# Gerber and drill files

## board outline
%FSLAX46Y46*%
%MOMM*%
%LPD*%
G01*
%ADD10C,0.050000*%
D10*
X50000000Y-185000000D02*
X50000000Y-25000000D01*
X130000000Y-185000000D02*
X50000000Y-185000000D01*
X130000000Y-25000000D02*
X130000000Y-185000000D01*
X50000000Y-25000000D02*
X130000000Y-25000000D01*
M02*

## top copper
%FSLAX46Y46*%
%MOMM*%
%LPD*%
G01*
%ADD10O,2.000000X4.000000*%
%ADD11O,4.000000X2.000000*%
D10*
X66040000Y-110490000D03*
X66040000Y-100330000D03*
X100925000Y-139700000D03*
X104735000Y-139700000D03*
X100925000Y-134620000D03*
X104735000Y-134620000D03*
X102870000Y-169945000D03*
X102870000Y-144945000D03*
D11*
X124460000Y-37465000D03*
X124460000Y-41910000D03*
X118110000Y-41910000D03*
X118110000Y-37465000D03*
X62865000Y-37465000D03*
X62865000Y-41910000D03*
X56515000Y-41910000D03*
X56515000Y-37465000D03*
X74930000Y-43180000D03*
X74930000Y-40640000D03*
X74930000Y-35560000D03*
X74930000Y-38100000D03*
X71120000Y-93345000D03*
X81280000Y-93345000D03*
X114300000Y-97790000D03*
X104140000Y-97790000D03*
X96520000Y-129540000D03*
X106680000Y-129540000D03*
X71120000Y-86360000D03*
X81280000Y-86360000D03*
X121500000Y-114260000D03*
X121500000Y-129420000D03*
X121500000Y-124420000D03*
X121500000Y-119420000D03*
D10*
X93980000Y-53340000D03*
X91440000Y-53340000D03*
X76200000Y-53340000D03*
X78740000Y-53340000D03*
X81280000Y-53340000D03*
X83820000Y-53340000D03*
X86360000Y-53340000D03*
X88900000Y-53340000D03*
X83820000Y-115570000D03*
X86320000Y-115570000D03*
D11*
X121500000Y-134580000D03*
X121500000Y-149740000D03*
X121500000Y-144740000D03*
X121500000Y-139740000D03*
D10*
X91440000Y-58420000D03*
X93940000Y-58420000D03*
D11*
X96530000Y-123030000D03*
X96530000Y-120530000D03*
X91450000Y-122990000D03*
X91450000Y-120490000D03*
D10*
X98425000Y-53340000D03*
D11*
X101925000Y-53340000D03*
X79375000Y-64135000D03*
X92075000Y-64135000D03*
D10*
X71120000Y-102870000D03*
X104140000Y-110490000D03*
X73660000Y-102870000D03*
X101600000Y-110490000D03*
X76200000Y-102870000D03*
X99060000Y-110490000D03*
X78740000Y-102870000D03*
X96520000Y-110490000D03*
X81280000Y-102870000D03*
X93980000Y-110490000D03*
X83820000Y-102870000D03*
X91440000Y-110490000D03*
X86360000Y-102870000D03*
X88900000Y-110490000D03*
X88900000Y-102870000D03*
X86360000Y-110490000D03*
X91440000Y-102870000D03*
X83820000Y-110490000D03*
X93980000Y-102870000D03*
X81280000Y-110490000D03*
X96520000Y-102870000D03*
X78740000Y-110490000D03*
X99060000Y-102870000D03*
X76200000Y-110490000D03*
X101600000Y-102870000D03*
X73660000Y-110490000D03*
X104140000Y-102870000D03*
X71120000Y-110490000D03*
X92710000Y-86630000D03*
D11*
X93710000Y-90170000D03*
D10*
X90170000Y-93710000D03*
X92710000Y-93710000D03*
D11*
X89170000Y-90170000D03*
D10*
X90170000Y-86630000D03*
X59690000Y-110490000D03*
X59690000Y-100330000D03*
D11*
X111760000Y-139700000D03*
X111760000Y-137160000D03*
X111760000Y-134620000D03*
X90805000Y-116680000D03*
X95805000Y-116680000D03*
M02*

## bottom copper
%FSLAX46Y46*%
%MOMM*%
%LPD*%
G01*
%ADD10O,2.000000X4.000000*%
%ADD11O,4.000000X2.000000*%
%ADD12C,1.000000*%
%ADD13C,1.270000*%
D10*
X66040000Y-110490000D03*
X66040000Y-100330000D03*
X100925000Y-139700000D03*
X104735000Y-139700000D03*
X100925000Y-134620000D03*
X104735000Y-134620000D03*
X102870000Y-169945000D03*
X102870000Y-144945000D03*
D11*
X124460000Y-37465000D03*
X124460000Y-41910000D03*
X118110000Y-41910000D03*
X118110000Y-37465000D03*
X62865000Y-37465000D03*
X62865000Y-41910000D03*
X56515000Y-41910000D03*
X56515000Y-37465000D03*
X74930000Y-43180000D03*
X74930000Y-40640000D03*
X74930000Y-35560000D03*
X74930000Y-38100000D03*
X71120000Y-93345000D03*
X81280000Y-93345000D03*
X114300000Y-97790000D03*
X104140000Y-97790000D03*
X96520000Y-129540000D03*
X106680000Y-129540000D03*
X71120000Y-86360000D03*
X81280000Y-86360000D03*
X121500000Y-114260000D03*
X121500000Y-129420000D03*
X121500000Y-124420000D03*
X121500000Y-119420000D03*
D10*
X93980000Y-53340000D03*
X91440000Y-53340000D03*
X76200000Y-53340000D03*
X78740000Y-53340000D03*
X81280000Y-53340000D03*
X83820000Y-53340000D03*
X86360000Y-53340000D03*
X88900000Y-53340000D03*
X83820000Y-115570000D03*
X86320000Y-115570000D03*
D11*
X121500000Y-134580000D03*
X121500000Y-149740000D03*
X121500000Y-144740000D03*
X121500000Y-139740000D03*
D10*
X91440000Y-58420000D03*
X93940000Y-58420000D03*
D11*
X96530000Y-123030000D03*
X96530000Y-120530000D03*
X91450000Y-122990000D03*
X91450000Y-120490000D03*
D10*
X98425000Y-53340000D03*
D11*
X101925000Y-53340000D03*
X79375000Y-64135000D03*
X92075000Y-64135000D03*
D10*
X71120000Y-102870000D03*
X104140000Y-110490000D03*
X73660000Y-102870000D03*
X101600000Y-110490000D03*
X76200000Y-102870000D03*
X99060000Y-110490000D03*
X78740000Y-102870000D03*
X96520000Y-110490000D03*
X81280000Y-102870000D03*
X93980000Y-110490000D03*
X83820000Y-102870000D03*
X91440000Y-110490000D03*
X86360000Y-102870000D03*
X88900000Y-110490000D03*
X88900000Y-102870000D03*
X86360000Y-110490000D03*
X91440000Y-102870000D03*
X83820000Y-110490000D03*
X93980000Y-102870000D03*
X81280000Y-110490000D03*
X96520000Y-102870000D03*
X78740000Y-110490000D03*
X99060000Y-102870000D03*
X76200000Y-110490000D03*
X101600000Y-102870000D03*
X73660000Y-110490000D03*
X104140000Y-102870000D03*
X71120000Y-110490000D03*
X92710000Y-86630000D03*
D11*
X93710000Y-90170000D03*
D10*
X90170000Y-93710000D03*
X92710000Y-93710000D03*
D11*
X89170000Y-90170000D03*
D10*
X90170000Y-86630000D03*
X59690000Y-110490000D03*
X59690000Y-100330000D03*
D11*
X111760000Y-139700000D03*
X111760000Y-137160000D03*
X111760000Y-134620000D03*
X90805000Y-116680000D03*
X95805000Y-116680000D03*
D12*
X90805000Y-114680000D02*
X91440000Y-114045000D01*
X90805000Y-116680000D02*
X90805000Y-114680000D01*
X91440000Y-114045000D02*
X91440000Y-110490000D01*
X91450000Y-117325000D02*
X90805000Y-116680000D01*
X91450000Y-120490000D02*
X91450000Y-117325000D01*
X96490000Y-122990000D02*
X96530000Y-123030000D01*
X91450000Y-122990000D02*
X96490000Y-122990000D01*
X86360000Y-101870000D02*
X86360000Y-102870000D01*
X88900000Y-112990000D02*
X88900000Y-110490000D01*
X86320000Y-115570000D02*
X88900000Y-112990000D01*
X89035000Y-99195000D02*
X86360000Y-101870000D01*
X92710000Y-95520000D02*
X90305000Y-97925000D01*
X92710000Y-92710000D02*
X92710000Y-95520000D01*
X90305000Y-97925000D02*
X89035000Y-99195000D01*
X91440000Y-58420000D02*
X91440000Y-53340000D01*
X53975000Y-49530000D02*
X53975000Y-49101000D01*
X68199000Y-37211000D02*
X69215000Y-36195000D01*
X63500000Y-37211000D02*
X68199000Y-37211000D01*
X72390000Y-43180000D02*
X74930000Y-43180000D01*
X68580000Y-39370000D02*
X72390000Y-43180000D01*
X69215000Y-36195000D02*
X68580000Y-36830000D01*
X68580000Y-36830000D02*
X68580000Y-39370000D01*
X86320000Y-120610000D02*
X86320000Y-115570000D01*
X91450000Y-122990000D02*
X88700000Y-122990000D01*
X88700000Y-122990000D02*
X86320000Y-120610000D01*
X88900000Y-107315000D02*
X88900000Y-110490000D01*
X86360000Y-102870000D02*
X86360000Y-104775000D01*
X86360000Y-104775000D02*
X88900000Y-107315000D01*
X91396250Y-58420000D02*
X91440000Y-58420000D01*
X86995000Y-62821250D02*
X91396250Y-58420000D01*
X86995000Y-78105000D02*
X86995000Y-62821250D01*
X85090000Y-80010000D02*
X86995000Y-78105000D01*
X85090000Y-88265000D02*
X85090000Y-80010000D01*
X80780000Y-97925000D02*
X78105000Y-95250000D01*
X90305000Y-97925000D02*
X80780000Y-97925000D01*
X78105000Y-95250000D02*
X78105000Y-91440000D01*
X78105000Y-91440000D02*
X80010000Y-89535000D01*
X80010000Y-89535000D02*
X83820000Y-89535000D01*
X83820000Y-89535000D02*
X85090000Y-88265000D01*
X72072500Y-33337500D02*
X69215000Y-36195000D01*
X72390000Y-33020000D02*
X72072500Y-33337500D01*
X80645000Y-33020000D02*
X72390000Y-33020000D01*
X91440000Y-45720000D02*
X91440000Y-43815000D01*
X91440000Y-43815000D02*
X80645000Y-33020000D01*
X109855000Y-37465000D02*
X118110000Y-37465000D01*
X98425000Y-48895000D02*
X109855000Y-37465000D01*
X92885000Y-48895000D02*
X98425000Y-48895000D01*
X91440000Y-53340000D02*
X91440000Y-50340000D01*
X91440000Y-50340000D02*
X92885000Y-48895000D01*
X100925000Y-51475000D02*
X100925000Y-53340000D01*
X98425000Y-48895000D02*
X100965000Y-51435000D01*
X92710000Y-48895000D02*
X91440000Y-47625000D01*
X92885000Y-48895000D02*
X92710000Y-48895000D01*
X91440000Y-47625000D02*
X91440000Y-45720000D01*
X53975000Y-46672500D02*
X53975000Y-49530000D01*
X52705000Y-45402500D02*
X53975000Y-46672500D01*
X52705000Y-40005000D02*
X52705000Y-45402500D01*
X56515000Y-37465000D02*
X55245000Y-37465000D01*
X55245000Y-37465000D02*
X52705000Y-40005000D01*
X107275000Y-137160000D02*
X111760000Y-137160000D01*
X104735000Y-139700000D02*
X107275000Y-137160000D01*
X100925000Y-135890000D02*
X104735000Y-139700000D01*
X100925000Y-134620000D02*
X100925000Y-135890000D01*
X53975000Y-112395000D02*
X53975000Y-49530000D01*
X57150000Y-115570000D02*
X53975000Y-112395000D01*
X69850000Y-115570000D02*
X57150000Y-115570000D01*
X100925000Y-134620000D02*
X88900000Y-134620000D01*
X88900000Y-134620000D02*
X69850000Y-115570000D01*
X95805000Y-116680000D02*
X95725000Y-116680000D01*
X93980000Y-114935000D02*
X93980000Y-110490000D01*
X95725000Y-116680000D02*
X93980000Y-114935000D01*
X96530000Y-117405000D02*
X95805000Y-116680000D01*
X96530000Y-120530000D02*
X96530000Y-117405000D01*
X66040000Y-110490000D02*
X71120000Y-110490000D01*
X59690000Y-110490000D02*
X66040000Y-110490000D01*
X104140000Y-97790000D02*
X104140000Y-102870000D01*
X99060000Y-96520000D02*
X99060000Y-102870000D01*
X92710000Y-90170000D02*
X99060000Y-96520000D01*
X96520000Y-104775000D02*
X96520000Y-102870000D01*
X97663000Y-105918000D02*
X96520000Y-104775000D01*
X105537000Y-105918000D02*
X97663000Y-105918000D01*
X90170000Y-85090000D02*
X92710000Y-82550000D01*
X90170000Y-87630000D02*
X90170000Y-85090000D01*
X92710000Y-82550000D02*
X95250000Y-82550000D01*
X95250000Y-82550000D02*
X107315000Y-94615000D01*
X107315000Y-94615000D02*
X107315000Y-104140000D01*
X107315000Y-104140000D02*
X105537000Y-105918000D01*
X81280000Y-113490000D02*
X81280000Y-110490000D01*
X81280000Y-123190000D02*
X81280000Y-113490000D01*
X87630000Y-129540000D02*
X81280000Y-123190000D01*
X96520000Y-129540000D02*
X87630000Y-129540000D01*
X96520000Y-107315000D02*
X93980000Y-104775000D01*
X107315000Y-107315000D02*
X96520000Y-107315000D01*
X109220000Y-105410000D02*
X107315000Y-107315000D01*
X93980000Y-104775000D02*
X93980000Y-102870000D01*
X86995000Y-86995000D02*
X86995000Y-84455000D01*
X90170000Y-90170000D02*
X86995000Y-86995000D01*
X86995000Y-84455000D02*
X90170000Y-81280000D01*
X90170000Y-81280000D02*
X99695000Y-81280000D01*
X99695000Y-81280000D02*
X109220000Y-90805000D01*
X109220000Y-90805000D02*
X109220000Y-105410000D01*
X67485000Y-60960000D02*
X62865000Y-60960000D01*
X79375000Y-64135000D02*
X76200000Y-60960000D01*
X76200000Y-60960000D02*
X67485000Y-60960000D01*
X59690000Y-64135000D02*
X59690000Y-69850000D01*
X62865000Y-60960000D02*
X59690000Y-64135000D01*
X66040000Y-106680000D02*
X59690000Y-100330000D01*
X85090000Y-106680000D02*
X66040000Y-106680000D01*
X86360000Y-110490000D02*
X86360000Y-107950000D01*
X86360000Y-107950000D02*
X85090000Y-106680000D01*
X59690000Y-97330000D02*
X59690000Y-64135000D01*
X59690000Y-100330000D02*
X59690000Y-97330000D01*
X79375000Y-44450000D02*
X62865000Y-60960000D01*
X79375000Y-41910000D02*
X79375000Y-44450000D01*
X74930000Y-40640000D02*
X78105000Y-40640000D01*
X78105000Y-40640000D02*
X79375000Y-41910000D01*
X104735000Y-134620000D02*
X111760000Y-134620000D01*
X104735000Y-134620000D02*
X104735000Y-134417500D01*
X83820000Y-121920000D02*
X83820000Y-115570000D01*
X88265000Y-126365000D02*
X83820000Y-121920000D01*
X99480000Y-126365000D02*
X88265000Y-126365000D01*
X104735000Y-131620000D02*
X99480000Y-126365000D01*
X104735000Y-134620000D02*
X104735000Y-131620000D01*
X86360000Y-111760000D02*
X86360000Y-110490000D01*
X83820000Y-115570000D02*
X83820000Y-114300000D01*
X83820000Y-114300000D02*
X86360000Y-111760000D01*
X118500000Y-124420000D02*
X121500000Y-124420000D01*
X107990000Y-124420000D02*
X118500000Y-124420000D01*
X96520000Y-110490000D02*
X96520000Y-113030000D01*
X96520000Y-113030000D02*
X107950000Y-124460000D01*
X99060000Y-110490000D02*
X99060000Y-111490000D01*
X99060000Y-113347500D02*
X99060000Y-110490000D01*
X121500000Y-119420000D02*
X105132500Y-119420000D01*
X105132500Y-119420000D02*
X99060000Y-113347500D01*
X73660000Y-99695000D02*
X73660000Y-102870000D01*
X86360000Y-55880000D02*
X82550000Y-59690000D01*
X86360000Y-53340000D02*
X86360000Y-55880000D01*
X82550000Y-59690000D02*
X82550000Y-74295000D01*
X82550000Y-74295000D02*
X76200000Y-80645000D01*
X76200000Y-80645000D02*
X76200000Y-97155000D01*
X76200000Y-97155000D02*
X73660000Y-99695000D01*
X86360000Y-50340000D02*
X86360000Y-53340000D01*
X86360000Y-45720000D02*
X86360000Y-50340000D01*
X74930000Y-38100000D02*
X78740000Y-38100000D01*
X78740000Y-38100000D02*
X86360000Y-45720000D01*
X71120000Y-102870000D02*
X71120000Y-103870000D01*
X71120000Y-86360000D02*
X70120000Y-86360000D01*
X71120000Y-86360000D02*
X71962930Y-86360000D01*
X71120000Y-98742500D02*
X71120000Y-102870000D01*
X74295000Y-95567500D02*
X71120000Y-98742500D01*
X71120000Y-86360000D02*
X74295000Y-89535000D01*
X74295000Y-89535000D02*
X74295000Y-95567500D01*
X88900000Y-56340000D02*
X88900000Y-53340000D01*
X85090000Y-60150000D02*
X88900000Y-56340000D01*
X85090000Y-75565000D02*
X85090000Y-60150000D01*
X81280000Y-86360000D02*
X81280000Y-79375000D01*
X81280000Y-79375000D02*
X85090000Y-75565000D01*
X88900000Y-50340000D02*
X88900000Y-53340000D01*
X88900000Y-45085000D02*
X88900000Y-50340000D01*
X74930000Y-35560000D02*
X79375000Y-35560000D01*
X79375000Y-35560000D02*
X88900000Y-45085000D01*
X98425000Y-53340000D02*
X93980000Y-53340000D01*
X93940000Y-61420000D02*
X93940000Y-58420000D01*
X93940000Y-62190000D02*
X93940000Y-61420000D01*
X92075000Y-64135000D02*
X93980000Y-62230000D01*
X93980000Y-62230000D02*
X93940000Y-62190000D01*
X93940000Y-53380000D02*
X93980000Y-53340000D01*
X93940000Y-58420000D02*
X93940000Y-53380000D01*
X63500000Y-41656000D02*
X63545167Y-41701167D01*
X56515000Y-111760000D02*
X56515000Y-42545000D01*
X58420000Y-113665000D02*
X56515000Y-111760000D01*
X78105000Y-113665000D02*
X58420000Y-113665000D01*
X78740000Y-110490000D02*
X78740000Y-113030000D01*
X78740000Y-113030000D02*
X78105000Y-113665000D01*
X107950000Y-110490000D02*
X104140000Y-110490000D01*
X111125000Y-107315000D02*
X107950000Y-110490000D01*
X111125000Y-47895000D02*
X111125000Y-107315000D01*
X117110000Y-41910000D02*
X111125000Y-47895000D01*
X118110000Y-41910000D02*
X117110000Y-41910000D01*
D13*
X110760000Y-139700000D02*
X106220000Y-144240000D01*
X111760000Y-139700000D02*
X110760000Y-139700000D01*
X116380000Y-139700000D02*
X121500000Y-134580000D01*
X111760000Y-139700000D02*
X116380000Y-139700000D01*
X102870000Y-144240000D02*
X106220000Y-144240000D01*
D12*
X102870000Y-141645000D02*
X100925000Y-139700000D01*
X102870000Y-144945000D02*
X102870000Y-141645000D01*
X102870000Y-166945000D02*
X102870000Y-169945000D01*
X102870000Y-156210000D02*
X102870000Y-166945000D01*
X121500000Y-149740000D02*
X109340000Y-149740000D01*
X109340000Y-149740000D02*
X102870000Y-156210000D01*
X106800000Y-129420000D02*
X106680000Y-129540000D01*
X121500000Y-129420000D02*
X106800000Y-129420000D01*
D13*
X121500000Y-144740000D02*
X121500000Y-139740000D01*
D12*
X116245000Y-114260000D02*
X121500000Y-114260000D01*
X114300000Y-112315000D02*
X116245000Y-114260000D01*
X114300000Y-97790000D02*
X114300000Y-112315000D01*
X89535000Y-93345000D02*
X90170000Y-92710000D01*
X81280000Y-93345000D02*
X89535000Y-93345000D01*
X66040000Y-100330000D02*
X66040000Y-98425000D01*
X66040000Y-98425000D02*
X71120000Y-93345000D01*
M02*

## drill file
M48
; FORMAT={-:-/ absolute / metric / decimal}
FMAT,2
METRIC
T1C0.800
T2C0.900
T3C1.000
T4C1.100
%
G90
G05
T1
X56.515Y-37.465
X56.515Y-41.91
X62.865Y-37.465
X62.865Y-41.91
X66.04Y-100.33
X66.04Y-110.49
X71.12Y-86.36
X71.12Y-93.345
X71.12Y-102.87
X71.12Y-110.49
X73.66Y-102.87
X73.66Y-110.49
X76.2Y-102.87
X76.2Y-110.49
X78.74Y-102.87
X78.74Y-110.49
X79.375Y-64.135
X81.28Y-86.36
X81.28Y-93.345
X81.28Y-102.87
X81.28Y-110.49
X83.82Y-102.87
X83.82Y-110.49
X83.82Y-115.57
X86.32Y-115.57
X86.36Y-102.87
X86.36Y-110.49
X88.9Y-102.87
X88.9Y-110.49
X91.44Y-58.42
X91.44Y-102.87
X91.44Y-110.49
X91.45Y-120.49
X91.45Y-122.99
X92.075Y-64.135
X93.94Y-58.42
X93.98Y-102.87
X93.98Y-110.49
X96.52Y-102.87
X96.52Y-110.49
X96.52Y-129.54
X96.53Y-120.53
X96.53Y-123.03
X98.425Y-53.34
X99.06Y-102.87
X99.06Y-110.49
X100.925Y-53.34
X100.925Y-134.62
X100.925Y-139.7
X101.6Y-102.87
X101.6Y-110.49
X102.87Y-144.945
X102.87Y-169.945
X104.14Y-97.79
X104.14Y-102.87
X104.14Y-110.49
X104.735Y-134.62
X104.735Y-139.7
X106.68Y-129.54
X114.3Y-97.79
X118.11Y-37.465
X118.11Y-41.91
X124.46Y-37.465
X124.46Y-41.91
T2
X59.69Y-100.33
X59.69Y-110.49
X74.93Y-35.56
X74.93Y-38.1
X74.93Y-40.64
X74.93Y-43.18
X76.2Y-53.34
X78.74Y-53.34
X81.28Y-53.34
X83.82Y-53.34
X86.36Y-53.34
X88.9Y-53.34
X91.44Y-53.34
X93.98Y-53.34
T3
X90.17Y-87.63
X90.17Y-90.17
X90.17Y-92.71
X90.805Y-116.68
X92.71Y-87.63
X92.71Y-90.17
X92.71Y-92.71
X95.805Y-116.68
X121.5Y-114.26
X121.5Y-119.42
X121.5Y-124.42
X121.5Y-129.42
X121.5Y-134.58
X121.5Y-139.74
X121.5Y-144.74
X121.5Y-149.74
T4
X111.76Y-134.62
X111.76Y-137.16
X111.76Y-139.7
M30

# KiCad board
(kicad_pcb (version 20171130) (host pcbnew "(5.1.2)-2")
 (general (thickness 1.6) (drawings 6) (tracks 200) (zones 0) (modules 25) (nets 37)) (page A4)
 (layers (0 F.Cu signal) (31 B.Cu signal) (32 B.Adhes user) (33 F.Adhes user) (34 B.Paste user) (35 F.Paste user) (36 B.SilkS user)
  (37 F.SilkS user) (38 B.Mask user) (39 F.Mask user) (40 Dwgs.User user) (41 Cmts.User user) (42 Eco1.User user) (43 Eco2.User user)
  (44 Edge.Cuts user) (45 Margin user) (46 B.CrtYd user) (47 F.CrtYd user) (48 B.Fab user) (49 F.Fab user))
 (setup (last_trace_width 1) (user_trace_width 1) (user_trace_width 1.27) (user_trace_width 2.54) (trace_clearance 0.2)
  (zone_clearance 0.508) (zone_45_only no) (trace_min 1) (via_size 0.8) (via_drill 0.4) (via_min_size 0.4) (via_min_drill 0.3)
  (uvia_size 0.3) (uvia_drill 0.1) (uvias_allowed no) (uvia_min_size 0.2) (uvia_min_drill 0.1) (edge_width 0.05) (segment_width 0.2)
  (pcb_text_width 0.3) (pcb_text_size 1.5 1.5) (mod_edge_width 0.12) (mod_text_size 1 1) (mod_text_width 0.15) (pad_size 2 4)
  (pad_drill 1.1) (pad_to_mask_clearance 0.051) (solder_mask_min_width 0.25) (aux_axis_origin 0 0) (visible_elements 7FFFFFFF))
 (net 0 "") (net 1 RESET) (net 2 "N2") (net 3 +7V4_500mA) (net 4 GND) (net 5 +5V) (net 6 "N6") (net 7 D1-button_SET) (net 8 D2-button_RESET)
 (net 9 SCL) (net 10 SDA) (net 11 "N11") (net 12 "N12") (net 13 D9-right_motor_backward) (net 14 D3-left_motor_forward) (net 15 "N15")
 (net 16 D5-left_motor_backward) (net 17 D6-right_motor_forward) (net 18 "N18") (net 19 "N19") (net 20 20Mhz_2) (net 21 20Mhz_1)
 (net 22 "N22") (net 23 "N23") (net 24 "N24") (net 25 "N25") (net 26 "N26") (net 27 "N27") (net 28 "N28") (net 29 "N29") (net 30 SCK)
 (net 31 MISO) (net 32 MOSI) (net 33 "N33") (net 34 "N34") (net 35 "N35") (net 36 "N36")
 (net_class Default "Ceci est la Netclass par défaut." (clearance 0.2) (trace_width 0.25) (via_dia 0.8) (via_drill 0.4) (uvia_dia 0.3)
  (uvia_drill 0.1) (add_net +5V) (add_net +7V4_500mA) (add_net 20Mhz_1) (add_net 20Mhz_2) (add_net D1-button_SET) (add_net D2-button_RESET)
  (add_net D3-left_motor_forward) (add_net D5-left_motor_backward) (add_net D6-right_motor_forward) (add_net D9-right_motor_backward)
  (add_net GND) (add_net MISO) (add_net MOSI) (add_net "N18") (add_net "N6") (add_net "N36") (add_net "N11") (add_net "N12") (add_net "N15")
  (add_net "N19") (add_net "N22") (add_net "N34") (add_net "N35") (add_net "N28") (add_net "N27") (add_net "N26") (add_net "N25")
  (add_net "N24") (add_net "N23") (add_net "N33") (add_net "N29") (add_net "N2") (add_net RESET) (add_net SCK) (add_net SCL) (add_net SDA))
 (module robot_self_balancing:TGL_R (layer F.Cu) (at 66.04 100.33 270)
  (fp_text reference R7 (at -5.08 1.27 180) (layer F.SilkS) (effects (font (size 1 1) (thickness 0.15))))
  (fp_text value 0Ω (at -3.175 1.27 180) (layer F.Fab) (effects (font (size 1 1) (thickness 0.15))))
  (pad 2 thru_hole oval (at 10.16 0 270) (size 4 2) (drill 0.8) (layers *.Cu *.Mask) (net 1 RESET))
  (pad 1 thru_hole oval (at 0 0 270) (size 4 2) (drill 0.8) (layers *.Cu *.Mask) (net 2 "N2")))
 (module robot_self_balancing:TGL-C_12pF (layer F.Cu) (at 104.1 139.7 180)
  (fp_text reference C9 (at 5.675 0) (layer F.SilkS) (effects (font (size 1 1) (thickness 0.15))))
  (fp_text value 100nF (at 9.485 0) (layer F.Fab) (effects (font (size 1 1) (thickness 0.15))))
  (pad 2 thru_hole oval (at 3.175 0 180) (size 2 4) (drill 0.8) (layers *.Cu *.Mask) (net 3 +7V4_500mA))
  (pad 1 thru_hole oval (at -0.635 0 180) (size 2 4) (drill 0.8) (layers *.Cu *.Mask) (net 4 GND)))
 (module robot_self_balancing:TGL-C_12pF (layer F.Cu) (at 104.1 134.62 180)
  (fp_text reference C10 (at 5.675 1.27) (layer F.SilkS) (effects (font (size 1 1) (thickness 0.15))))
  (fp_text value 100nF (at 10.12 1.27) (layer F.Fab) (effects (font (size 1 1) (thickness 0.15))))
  (pad 2 thru_hole oval (at 3.175 0 180) (size 2 4) (drill 0.8) (layers *.Cu *.Mask) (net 4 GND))
  (pad 1 thru_hole oval (at -0.635 0 180) (size 2 4) (drill 0.8) (layers *.Cu *.Mask) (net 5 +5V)))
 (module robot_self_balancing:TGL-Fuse (layer F.Cu) (at 111.76 156.845 270)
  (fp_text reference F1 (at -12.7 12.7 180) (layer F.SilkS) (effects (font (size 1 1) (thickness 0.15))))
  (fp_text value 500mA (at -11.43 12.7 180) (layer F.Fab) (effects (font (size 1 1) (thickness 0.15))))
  (pad 2 thru_hole oval (at 13.1 8.89 270) (size 4 2) (drill 0.8) (layers *.Cu *.Mask) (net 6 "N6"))
  (pad 1 thru_hole oval (at -11.9 8.89 270) (size 4 2) (drill 0.8) (layers *.Cu *.Mask) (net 3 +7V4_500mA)))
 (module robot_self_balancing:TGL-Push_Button (layer F.Cu) (at 121.285 34.925)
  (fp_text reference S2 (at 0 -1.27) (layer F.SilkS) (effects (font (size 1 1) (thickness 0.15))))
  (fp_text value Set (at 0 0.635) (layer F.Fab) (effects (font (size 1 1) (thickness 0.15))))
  (pad 1 thru_hole oval (at 3.175 2.54) (size 4 2) (drill 0.8) (layers *.Cu *.Mask) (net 4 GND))
  (pad 2 thru_hole oval (at 3.175 6.985) (size 4 2) (drill 0.8) (layers *.Cu *.Mask) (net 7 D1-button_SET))
  (pad 2 thru_hole oval (at -3.175 6.985) (size 4 2) (drill 0.8) (layers *.Cu *.Mask) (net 7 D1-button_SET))
  (pad 1 thru_hole oval (at -3.175 2.54) (size 4 2) (drill 0.8) (layers *.Cu *.Mask) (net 4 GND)))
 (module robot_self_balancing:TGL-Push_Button (layer F.Cu) (at 59.69 34.925)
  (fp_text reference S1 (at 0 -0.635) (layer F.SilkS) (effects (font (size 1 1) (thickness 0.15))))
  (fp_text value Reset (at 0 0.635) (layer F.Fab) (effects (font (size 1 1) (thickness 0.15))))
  (pad 1 thru_hole oval (at 3.175 2.54) (size 4 2) (drill 0.8) (layers *.Cu *.Mask) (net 4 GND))
  (pad 2 thru_hole oval (at 3.175 6.985) (size 4 2) (drill 0.8) (layers *.Cu *.Mask) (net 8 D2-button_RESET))
  (pad 2 thru_hole oval (at -3.175 6.985) (size 4 2) (drill 0.8) (layers *.Cu *.Mask) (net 8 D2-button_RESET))
  (pad 1 thru_hole oval (at -3.175 2.54) (size 4 2) (drill 0.8) (layers *.Cu *.Mask) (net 4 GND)))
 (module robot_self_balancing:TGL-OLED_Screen (layer F.Cu) (at 71.12 39.37 90)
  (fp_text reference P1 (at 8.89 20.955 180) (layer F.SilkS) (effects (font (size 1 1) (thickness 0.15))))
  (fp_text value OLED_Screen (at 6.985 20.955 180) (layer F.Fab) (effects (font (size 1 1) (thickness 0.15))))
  (pad 1 thru_hole oval (at -3.81 3.81 90) (size 2 4) (drill 0.9) (layers *.Cu *.Mask) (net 4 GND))
  (pad 2 thru_hole oval (at -1.27 3.81 90) (size 2 4) (drill 0.9) (layers *.Cu *.Mask) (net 5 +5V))
  (pad 4 thru_hole oval (at 3.81 3.81 90) (size 2 4) (drill 0.9) (layers *.Cu *.Mask) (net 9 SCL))
  (pad 3 thru_hole oval (at 1.27 3.81 90) (size 2 4) (drill 0.9) (layers *.Cu *.Mask) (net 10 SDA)))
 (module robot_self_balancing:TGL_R (layer F.Cu) (at 81.28 93.345 180)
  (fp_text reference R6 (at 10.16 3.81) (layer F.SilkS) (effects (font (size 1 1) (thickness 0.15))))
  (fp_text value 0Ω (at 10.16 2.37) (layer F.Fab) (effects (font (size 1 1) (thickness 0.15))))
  (pad 2 thru_hole oval (at 10.16 0 180) (size 4 2) (drill 0.8) (layers *.Cu *.Mask) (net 2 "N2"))
  (pad 1 thru_hole oval (at 0 0 180) (size 4 2) (drill 0.8) (layers *.Cu *.Mask) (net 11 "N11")))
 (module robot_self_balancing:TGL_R (layer F.Cu) (at 104.14 97.79)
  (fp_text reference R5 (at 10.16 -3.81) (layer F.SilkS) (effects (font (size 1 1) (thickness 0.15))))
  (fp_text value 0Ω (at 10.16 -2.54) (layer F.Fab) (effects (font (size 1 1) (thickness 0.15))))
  (pad 2 thru_hole oval (at 10.16 0) (size 4 2) (drill 0.8) (layers *.Cu *.Mask) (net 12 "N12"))
  (pad 1 thru_hole oval (at 0 0) (size 4 2) (drill 0.8) (layers *.Cu *.Mask) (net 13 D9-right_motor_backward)))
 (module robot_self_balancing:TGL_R (layer F.Cu) (at 106.68 129.54 180)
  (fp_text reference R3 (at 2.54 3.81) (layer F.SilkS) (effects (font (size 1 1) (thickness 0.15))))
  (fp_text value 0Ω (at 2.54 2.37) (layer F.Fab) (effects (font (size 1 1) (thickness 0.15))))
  (pad 2 thru_hole oval (at 10.16 0 180) (size 4 2) (drill 0.8) (layers *.Cu *.Mask) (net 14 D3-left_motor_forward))
  (pad 1 thru_hole oval (at 0 0 180) (size 4 2) (drill 0.8) (layers *.Cu *.Mask) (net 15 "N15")))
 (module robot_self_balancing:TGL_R (layer F.Cu) (at 81.28 86.36 180)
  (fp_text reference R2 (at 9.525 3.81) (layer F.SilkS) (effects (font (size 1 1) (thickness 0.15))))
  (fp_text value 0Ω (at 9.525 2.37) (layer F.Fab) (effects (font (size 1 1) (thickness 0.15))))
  (pad 2 thru_hole oval (at 10.16 0 180) (size 4 2) (drill 0.8) (layers *.Cu *.Mask) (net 9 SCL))
  (pad 1 thru_hole oval (at 0 0 180) (size 4 2) (drill 0.8) (layers *.Cu *.Mask) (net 9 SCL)))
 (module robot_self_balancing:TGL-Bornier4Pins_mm (layer F.Cu) (at 127 121.92 270)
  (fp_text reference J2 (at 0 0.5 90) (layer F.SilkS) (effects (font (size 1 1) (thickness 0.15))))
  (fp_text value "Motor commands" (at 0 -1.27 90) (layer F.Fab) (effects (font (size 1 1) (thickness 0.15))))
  (pad 5 thru_hole oval (at -7.66 5.5 270) (size 2 4) (drill 1) (layers *.Cu *.Mask) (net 12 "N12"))
  (pad 8 thru_hole oval (at 7.5 5.5 90) (size 2 4) (drill 1) (layers *.Cu *.Mask) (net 15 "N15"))
  (pad 7 thru_hole oval (at 2.5 5.5 270) (size 2 4) (drill 1) (layers *.Cu *.Mask) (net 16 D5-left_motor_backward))
  (pad 6 thru_hole oval (at -2.5 5.5 270) (size 2 4) (drill 1) (layers *.Cu *.Mask) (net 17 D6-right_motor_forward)))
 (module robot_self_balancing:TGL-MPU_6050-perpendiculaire (layer F.Cu) (at 85.09 57.15 180)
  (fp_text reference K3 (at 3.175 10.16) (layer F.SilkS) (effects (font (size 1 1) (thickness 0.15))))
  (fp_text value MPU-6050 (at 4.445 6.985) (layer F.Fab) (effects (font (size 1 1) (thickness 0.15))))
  (pad 13 thru_hole oval (at -8.89 3.81 180) (size 2 4) (drill 0.9) (layers *.Cu *.Mask) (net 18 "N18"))
  (pad 18 thru_hole oval (at -6.35 3.81 180) (size 2 4) (drill 0.9) (layers *.Cu *.Mask) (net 4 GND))
  (pad "" thru_hole oval (at 8.89 3.81 180) (size 2 4) (drill 0.9) (layers *.Cu *.Mask))
  (pad "" thru_hole oval (at 6.35 3.81 180) (size 2 4) (drill 0.9) (layers *.Cu *.Mask))
  (pad "" thru_hole oval (at 3.81 3.81 180) (size 2 4) (drill 0.9) (layers *.Cu *.Mask))
  (pad "" thru_hole oval (at 1.27 3.81 180) (size 2 4) (drill 0.9) (layers *.Cu *.Mask))
  (pad 24 thru_hole oval (at -1.27 3.81 180) (size 2 4) (drill 0.9) (layers *.Cu *.Mask) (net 10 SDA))
  (pad 23 thru_hole oval (at -3.81 3.81 180) (size 2 4) (drill 0.9) (layers *.Cu *.Mask) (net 9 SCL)))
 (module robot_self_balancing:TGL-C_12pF (layer F.Cu) (at 86.32 115.57 180)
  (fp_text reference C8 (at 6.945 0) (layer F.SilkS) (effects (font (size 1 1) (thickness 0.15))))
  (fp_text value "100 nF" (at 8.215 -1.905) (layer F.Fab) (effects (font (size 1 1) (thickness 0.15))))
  (pad 2 thru_hole oval (at 2.5 0 180) (size 2 4) (drill 0.8) (layers *.Cu *.Mask) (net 5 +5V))
  (pad 1 thru_hole oval (at 0 0 180) (size 2 4) (drill 0.8) (layers *.Cu *.Mask) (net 4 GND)))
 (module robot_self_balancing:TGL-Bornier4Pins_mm (layer F.Cu) (at 127 142.24 270)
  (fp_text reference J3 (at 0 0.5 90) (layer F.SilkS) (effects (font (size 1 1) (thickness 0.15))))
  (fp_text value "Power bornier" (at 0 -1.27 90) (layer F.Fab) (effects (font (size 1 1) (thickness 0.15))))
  (pad 8 thru_hole oval (at -7.66 5.5 270) (size 2 4) (drill 1) (layers *.Cu *.Mask) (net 3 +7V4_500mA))
  (pad 5 thru_hole oval (at 7.5 5.5 90) (size 2 4) (drill 1) (layers *.Cu *.Mask) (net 6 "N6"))
  (pad 7 thru_hole oval (at 2.5 5.5 270) (size 2 4) (drill 1) (layers *.Cu *.Mask) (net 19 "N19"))
  (pad 6 thru_hole oval (at -2.5 5.5 270) (size 2 4) (drill 1) (layers *.Cu *.Mask) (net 19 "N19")))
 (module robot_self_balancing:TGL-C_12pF (layer F.Cu) (at 93.94 58.42 180)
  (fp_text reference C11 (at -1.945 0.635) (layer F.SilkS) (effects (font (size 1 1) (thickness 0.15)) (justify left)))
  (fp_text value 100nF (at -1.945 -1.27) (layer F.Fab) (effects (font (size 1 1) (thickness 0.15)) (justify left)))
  (pad 2 thru_hole oval (at 2.5 0 180) (size 2 4) (drill 0.8) (layers *.Cu *.Mask) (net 4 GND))
  (pad 1 thru_hole oval (at 0 0 180) (size 2 4) (drill 0.8) (layers *.Cu *.Mask) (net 18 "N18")))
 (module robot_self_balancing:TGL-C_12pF (layer F.Cu) (at 96.53 120.53 270)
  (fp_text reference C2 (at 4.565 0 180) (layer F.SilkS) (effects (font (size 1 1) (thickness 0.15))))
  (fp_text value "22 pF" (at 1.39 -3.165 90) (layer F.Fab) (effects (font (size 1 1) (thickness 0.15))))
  (pad 2 thru_hole oval (at 2.5 0 270) (size 2 4) (drill 0.8) (layers *.Cu *.Mask) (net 4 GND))
  (pad 1 thru_hole oval (at 0 0 270) (size 2 4) (drill 0.8) (layers *.Cu *.Mask) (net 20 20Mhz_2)))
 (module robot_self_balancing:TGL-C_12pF (layer F.Cu) (at 91.45 120.49 270)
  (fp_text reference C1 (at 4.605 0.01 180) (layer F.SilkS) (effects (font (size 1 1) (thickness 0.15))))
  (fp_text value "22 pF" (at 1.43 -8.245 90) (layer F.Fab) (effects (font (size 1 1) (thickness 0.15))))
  (pad 2 thru_hole oval (at 2.5 0 270) (size 2 4) (drill 0.8) (layers *.Cu *.Mask) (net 4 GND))
  (pad 1 thru_hole oval (at 0 0 270) (size 2 4) (drill 0.8) (layers *.Cu *.Mask) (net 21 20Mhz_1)))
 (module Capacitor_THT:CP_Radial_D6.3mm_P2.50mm (layer F.Cu) (at 98.425 53.34)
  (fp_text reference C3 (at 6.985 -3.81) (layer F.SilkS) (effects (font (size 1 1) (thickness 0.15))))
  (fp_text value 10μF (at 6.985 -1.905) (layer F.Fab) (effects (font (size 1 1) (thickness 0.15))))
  (pad 1 thru_hole oval (at 0 0) (size 2 4) (drill 0.8) (layers *.Cu *.Mask) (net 18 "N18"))
  (pad 2 thru_hole oval (at 2.5 0) (size 4 2) (drill 0.8 (offset 1 0)) (layers *.Cu *.Mask) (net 4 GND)))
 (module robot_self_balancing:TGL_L (layer F.Cu) (at 92.075 64.135 180)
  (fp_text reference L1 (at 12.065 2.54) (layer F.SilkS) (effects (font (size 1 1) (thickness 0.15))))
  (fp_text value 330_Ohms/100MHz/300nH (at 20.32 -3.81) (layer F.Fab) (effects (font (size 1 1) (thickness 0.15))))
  (pad 2 thru_hole oval (at 12.7 0 180) (size 4 2) (drill 0.8) (layers *.Cu *.Mask) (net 5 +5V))
  (pad 1 thru_hole oval (at 0 0 180) (size 4 2) (drill 0.8) (layers *.Cu *.Mask) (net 18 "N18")))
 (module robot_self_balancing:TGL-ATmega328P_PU (layer F.Cu) (at 71.12 110.49 90)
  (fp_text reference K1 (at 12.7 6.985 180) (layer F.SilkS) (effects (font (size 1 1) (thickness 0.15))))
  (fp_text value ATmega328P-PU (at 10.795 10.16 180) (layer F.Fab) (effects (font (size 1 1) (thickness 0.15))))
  (pad 28 thru_hole oval (at 7.62 0 90) (size 4 2) (drill 0.8) (layers *.Cu *.Mask) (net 9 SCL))
  (pad 14 thru_hole oval (at 0 33.02 90) (size 4 2) (drill 0.8) (layers *.Cu *.Mask) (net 7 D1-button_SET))
  (pad 27 thru_hole oval (at 7.62 2.54 90) (size 4 2) (drill 0.8) (layers *.Cu *.Mask) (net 10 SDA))
  (pad 13 thru_hole oval (at 0 30.48 90) (size 4 2) (drill 0.8) (layers *.Cu *.Mask) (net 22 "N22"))
  (pad 26 thru_hole oval (at 7.62 5.08 90) (size 4 2) (drill 0.8) (layers *.Cu *.Mask) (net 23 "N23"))
  (pad 12 thru_hole oval (at 0 27.94 90) (size 4 2) (drill 0.8) (layers *.Cu *.Mask) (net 17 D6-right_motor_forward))
  (pad 25 thru_hole oval (at 7.62 7.62 90) (size 4 2) (drill 0.8) (layers *.Cu *.Mask) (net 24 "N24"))
  (pad 11 thru_hole oval (at 0 25.4 90) (size 4 2) (drill 0.8) (layers *.Cu *.Mask) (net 16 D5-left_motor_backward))
  (pad 24 thru_hole oval (at 7.62 10.16 90) (size 4 2) (drill 0.8) (layers *.Cu *.Mask) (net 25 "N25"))
  (pad 10 thru_hole oval (at 0 22.86 90) (size 4 2) (drill 0.8) (layers *.Cu *.Mask) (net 20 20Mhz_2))
  (pad 23 thru_hole oval (at 7.62 12.7 90) (size 4 2) (drill 0.8) (layers *.Cu *.Mask) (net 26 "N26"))
  (pad 9 thru_hole oval (at 0 20.32 90) (size 4 2) (drill 0.8) (layers *.Cu *.Mask) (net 21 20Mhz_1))
  (pad 22 thru_hole oval (at 7.62 15.24 90) (size 4 2) (drill 0.8) (layers *.Cu *.Mask) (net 4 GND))
  (pad 8 thru_hole oval (at 0 17.78 90) (size 4 2) (drill 0.8) (layers *.Cu *.Mask) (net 4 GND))
  (pad 21 thru_hole oval (at 7.62 17.78 90) (size 4 2) (drill 0.8) (layers *.Cu *.Mask) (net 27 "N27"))
  (pad 7 thru_hole oval (at 0 15.24 90) (size 4 2) (drill 0.8) (layers *.Cu *.Mask) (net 5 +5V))
  (pad 20 thru_hole oval (at 7.62 20.32 90) (size 4 2) (drill 0.8) (layers *.Cu *.Mask) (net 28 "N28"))
  (pad 6 thru_hole oval (at 0 12.7 90) (size 4 2) (drill 0.8) (layers *.Cu *.Mask) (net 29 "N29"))
  (pad 19 thru_hole oval (at 7.62 22.86 90) (size 4 2) (drill 0.8) (layers *.Cu *.Mask) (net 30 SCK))
  (pad 5 thru_hole oval (at 0 10.16 90) (size 4 2) (drill 0.8) (layers *.Cu *.Mask) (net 14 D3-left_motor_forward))
  (pad 18 thru_hole oval (at 7.62 25.4 90) (size 4 2) (drill 0.8) (layers *.Cu *.Mask) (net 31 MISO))
  (pad 4 thru_hole oval (at 0 7.62 90) (size 4 2) (drill 0.8) (layers *.Cu *.Mask) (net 8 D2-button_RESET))
  (pad 17 thru_hole oval (at 7.62 27.94 90) (size 4 2) (drill 0.8) (layers *.Cu *.Mask) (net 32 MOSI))
  (pad 3 thru_hole oval (at 0 5.08 90) (size 4 2) (drill 0.8) (layers *.Cu *.Mask) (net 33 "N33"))
  (pad 16 thru_hole oval (at 7.62 30.48 90) (size 4 2) (drill 0.8) (layers *.Cu *.Mask) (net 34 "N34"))
  (pad 2 thru_hole oval (at 0 2.54 90) (size 4 2) (drill 0.8) (layers *.Cu *.Mask) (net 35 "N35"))
  (pad 15 thru_hole oval (at 7.62 33.02 90) (size 4 2) (drill 0.8) (layers *.Cu *.Mask) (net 13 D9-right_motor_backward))
  (pad 1 thru_hole oval (at 0 0 90) (size 4 2) (drill 0.8) (layers *.Cu *.Mask) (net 1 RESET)))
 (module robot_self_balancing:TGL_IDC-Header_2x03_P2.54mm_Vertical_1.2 (layer F.Cu) (at 90.17 87.63)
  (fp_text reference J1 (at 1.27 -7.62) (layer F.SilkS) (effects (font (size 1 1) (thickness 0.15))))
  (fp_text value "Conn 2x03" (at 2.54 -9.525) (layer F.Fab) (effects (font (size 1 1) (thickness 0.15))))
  (pad 2 thru_hole oval (at 2.54 0) (size 2 4) (drill 1 (offset 0 -1)) (layers *.Cu *.Mask) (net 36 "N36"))
  (pad 4 thru_hole oval (at 2.54 2.54) (size 4 2) (drill 1 (offset 1 0)) (layers *.Cu *.Mask) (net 32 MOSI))
  (pad 5 thru_hole oval (at 0 5.08) (size 2 4) (drill 1 (offset 0 1)) (layers *.Cu *.Mask) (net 11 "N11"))
  (pad 6 thru_hole oval (at 2.54 5.08) (size 2 4) (drill 1 (offset 0 1)) (layers *.Cu *.Mask) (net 4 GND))
  (pad 3 thru_hole oval (at 0 2.54) (size 4 2) (drill 1 (offset -1 0)) (layers *.Cu *.Mask) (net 30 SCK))
  (pad 1 thru_hole oval (at 0 0) (size 2 4) (drill 1 (offset 0 -1)) (layers *.Cu *.Mask) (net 31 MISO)))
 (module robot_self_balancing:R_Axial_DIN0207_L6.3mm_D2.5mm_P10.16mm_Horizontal (layer F.Cu) (at 59.69 100.33 270)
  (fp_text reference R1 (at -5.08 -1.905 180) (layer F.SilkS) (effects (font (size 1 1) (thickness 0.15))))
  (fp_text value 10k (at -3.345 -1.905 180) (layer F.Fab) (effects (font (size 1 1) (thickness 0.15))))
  (pad 2 thru_hole oval (at 10.16 0 270) (size 4 2) (drill 0.9) (layers *.Cu *.Mask) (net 1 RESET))
  (pad 1 thru_hole oval (at 0 0 270) (size 4 2) (drill 0.9) (layers *.Cu *.Mask) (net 5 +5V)))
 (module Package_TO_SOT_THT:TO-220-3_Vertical (layer F.Cu) (at 111.76 139.7 90)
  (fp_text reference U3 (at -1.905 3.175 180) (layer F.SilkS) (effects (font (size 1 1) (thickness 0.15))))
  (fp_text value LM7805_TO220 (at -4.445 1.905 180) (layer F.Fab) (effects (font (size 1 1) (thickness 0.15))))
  (pad 1 thru_hole oval (at 0 0 90) (size 2 4) (drill 1.1) (layers *.Cu *.Mask) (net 3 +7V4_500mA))
  (pad 2 thru_hole oval (at 2.54 0 90) (size 2 4) (drill 1.1) (layers *.Cu *.Mask) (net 4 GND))
  (pad 3 thru_hole oval (at 5.08 0 90) (size 2 4) (drill 1.1) (layers *.Cu *.Mask) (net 5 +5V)))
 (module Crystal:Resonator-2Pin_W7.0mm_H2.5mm (layer F.Cu) (at 90.805 116.68)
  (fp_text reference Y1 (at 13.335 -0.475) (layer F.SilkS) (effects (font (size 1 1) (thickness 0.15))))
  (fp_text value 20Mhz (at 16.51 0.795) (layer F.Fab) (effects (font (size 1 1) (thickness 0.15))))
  (pad 1 thru_hole oval (at 0 0) (size 4 2) (drill 1) (layers *.Cu *.Mask) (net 21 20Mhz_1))
  (pad 2 thru_hole oval (at 5 0) (size 4 2) (drill 1) (layers *.Cu *.Mask) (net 20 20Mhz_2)))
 (gr_line (start 50 185) (end 50 25) (layer Edge.Cuts) (width 0.05))
 (gr_line (start 130 185) (end 50 185) (layer Edge.Cuts) (width 0.05))
 (gr_line (start 130 25) (end 130 185) (layer Edge.Cuts) (width 0.05))
 (gr_line (start 50 25) (end 130 25) (layer Edge.Cuts) (width 0.05))
 (segment (start 90.805 114.68) (end 91.44 114.045) (width 1) (layer B.Cu) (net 21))
 (segment (start 90.805 116.68) (end 90.805 114.68) (width 1) (layer B.Cu) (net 21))
 (segment (start 91.44 114.045) (end 91.44 110.49) (width 1) (layer B.Cu) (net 21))
 (segment (start 91.45 117.325) (end 90.805 116.68) (width 1) (layer B.Cu) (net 21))
 (segment (start 91.45 120.49) (end 91.45 117.325) (width 1) (layer B.Cu) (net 21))
 (segment (start 96.49 122.99) (end 96.53 123.03) (width 1) (layer B.Cu) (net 4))
 (segment (start 91.45 122.99) (end 96.49 122.99) (width 1) (layer B.Cu) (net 4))
 (segment (start 86.36 101.87) (end 86.36 102.87) (width 1) (layer B.Cu) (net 4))
 (segment (start 88.9 112.99) (end 88.9 110.49) (width 1) (layer B.Cu) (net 4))
 (segment (start 86.32 115.57) (end 88.9 112.99) (width 1) (layer B.Cu) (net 4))
 (segment (start 89.035 99.195) (end 86.36 101.87) (width 1) (layer B.Cu) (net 4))
 (segment (start 92.71 95.52) (end 90.305 97.925) (width 1) (layer B.Cu) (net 4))
 (segment (start 92.71 92.71) (end 92.71 95.52) (width 1) (layer B.Cu) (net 4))
 (segment (start 90.305 97.925) (end 89.035 99.195) (width 1) (layer B.Cu) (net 4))
 (segment (start 91.44 58.42) (end 91.44 53.34) (width 1) (layer B.Cu) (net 4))
 (segment (start 53.975 49.53) (end 53.975 49.101) (width 1) (layer B.Cu) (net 4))
 (segment (start 68.199 37.211) (end 69.215 36.195) (width 1) (layer B.Cu) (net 4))
 (segment (start 63.5 37.211) (end 68.199 37.211) (width 1) (layer B.Cu) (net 4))
 (segment (start 72.39 43.18) (end 74.93 43.18) (width 1) (layer B.Cu) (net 4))
 (segment (start 68.58 39.37) (end 72.39 43.18) (width 1) (layer B.Cu) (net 4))
 (segment (start 69.215 36.195) (end 68.58 36.83) (width 1) (layer B.Cu) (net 4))
 (segment (start 68.58 36.83) (end 68.58 39.37) (width 1) (layer B.Cu) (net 4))
 (segment (start 86.32 120.61) (end 86.32 115.57) (width 1) (layer B.Cu) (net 4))
 (segment (start 91.45 122.99) (end 88.7 122.99) (width 1) (layer B.Cu) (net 4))
 (segment (start 88.7 122.99) (end 86.32 120.61) (width 1) (layer B.Cu) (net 4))
 (segment (start 88.9 107.315) (end 88.9 110.49) (width 1) (layer B.Cu) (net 4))
 (segment (start 86.36 102.87) (end 86.36 104.775) (width 1) (layer B.Cu) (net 4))
 (segment (start 86.36 104.775) (end 88.9 107.315) (width 1) (layer B.Cu) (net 4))
 (segment (start 91.39625 58.42) (end 91.44 58.42) (width 1) (layer B.Cu) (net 4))
 (segment (start 86.995 62.82125) (end 91.39625 58.42) (width 1) (layer B.Cu) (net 4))
 (segment (start 86.995 78.105) (end 86.995 62.82125) (width 1) (layer B.Cu) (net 4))
 (segment (start 85.09 80.01) (end 86.995 78.105) (width 1) (layer B.Cu) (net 4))
 (segment (start 85.09 88.265) (end 85.09 80.01) (width 1) (layer B.Cu) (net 4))
 (segment (start 80.78 97.925) (end 78.105 95.25) (width 1) (layer B.Cu) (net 4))
 (segment (start 90.305 97.925) (end 80.78 97.925) (width 1) (layer B.Cu) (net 4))
 (segment (start 78.105 95.25) (end 78.105 91.44) (width 1) (layer B.Cu) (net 4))
 (segment (start 78.105 91.44) (end 80.01 89.535) (width 1) (layer B.Cu) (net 4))
 (segment (start 80.01 89.535) (end 83.82 89.535) (width 1) (layer B.Cu) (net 4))
 (segment (start 83.82 89.535) (end 85.09 88.265) (width 1) (layer B.Cu) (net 4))
 (segment (start 72.0725 33.3375) (end 69.215 36.195) (width 1) (layer B.Cu) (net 4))
 (segment (start 72.39 33.02) (end 72.0725 33.3375) (width 1) (layer B.Cu) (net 4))
 (segment (start 80.645 33.02) (end 72.39 33.02) (width 1) (layer B.Cu) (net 4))
 (segment (start 91.44 45.72) (end 91.44 43.815) (width 1) (layer B.Cu) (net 4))
 (segment (start 91.44 43.815) (end 80.645 33.02) (width 1) (layer B.Cu) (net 4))
 (segment (start 109.855 37.465) (end 118.11 37.465) (width 1) (layer B.Cu) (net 4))
 (segment (start 98.425 48.895) (end 109.855 37.465) (width 1) (layer B.Cu) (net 4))
 (segment (start 92.885 48.895) (end 98.425 48.895) (width 1) (layer B.Cu) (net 4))
 (segment (start 91.44 53.34) (end 91.44 50.34) (width 1) (layer B.Cu) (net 4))
 (segment (start 91.44 50.34) (end 92.885 48.895) (width 1) (layer B.Cu) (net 4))
 (segment (start 100.925 51.475) (end 100.925 53.34) (width 1) (layer B.Cu) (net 4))
 (segment (start 98.425 48.895) (end 100.965 51.435) (width 1) (layer B.Cu) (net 4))
 (segment (start 92.71 48.895) (end 91.44 47.625) (width 1) (layer B.Cu) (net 4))
 (segment (start 92.885 48.895) (end 92.71 48.895) (width 1) (layer B.Cu) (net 4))
 (segment (start 91.44 47.625) (end 91.44 45.72) (width 1) (layer B.Cu) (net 4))
 (segment (start 53.975 46.6725) (end 53.975 49.53) (width 1) (layer B.Cu) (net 4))
 (segment (start 52.705 45.4025) (end 53.975 46.6725) (width 1) (layer B.Cu) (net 4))
 (segment (start 52.705 40.005) (end 52.705 45.4025) (width 1) (layer B.Cu) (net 4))
 (segment (start 56.515 37.465) (end 55.245 37.465) (width 1) (layer B.Cu) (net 4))
 (segment (start 55.245 37.465) (end 52.705 40.005) (width 1) (layer B.Cu) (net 4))
 (segment (start 107.275 137.16) (end 111.76 137.16) (width 1) (layer B.Cu) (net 4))
 (segment (start 104.735 139.7) (end 107.275 137.16) (width 1) (layer B.Cu) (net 4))
 (segment (start 100.925 135.89) (end 104.735 139.7) (width 1) (layer B.Cu) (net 4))
 (segment (start 100.925 134.62) (end 100.925 135.89) (width 1) (layer B.Cu) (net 4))
 (segment (start 53.975 112.395) (end 53.975 49.53) (width 1) (layer B.Cu) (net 4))
 (segment (start 57.15 115.57) (end 53.975 112.395) (width 1) (layer B.Cu) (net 4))
 (segment (start 69.85 115.57) (end 57.15 115.57) (width 1) (layer B.Cu) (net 4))
 (segment (start 100.925 134.62) (end 88.9 134.62) (width 1) (layer B.Cu) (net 4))
 (segment (start 88.9 134.62) (end 69.85 115.57) (width 1) (layer B.Cu) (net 4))
 (segment (start 95.805 116.68) (end 95.725 116.68) (width 1) (layer B.Cu) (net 20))
 (segment (start 93.98 114.935) (end 93.98 110.49) (width 1) (layer B.Cu) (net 20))
 (segment (start 95.725 116.68) (end 93.98 114.935) (width 1) (layer B.Cu) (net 20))
 (segment (start 96.53 117.405) (end 95.805 116.68) (width 1) (layer B.Cu) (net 20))
 (segment (start 96.53 120.53) (end 96.53 117.405) (width 1) (layer B.Cu) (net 20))
 (segment (start 66.04 110.49) (end 71.12 110.49) (width 1) (layer B.Cu) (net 1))
 (segment (start 59.69 110.49) (end 66.04 110.49) (width 1) (layer B.Cu) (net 1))
 (segment (start 104.14 97.79) (end 104.14 102.87) (width 1) (layer B.Cu) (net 13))
 (segment (start 99.06 96.52) (end 99.06 102.87) (width 1) (layer B.Cu) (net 32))
 (segment (start 92.71 90.17) (end 99.06 96.52) (width 1) (layer B.Cu) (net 32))
 (segment (start 96.52 104.775) (end 96.52 102.87) (width 1) (layer B.Cu) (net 31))
 (segment (start 97.663 105.918) (end 96.52 104.775) (width 1) (layer B.Cu) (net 31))
 (segment (start 105.537 105.918) (end 97.663 105.918) (width 1) (layer B.Cu) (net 31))
 (segment (start 90.17 85.09) (end 92.71 82.55) (width 1) (layer B.Cu) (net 31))
 (segment (start 90.17 87.63) (end 90.17 85.09) (width 1) (layer B.Cu) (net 31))
 (segment (start 92.71 82.55) (end 95.25 82.55) (width 1) (layer B.Cu) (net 31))
 (segment (start 95.25 82.55) (end 107.315 94.615) (width 1) (layer B.Cu) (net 31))
 (segment (start 107.315 94.615) (end 107.315 104.14) (width 1) (layer B.Cu) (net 31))
 (segment (start 107.315 104.14) (end 105.537 105.918) (width 1) (layer B.Cu) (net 31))
 (segment (start 81.28 113.49) (end 81.28 110.49) (width 1) (layer B.Cu) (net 14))
 (segment (start 81.28 123.19) (end 81.28 113.49) (width 1) (layer B.Cu) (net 14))
 (segment (start 87.63 129.54) (end 81.28 123.19) (width 1) (layer B.Cu) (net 14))
 (segment (start 96.52 129.54) (end 87.63 129.54) (width 1) (layer B.Cu) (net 14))
 (segment (start 96.52 107.315) (end 93.98 104.775) (width 1) (layer B.Cu) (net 30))
 (segment (start 107.315 107.315) (end 96.52 107.315) (width 1) (layer B.Cu) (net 30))
 (segment (start 109.22 105.41) (end 107.315 107.315) (width 1) (layer B.Cu) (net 30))
 (segment (start 93.98 104.775) (end 93.98 102.87) (width 1) (layer B.Cu) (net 30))
 (segment (start 86.995 86.995) (end 86.995 84.455) (width 1) (layer B.Cu) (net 30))
 (segment (start 90.17 90.17) (end 86.995 86.995) (width 1) (layer B.Cu) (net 30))
 (segment (start 86.995 84.455) (end 90.17 81.28) (width 1) (layer B.Cu) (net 30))
 (segment (start 90.17 81.28) (end 99.695 81.28) (width 1) (layer B.Cu) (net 30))
 (segment (start 99.695 81.28) (end 109.22 90.805) (width 1) (layer B.Cu) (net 30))
 (segment (start 109.22 90.805) (end 109.22 105.41) (width 1) (layer B.Cu) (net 30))
 (segment (start 67.485 60.96) (end 62.865 60.96) (width 1) (layer B.Cu) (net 5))
 (segment (start 79.375 64.135) (end 76.2 60.96) (width 1) (layer B.Cu) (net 5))
 (segment (start 76.2 60.96) (end 67.485 60.96) (width 1) (layer B.Cu) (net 5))
 (segment (start 59.69 64.135) (end 59.69 69.85) (width 1) (layer B.Cu) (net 5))
 (segment (start 62.865 60.96) (end 59.69 64.135) (width 1) (layer B.Cu) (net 5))
 (segment (start 66.04 106.68) (end 59.69 100.33) (width 1) (layer B.Cu) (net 5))
 (segment (start 85.09 106.68) (end 66.04 106.68) (width 1) (layer B.Cu) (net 5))
 (segment (start 86.36 110.49) (end 86.36 107.95) (width 1) (layer B.Cu) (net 5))
 (segment (start 86.36 107.95) (end 85.09 106.68) (width 1) (layer B.Cu) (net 5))
 (segment (start 59.69 97.33) (end 59.69 64.135) (width 1) (layer B.Cu) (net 5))
 (segment (start 59.69 100.33) (end 59.69 97.33) (width 1) (layer B.Cu) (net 5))
 (segment (start 79.375 44.45) (end 62.865 60.96) (width 1) (layer B.Cu) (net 5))
 (segment (start 79.375 41.91) (end 79.375 44.45) (width 1) (layer B.Cu) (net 5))
 (segment (start 74.93 40.64) (end 78.105 40.64) (width 1) (layer B.Cu) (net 5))
 (segment (start 78.105 40.64) (end 79.375 41.91) (width 1) (layer B.Cu) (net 5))
 (segment (start 104.735 134.62) (end 111.76 134.62) (width 1) (layer B.Cu) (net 5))
 (segment (start 104.735 134.62) (end 104.735 134.4175) (width 1) (layer B.Cu) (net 5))
 (segment (start 83.82 121.92) (end 83.82 115.57) (width 1) (layer B.Cu) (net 5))
 (segment (start 88.265 126.365) (end 83.82 121.92) (width 1) (layer B.Cu) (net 5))
 (segment (start 99.48 126.365) (end 88.265 126.365) (width 1) (layer B.Cu) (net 5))
 (segment (start 104.735 131.62) (end 99.48 126.365) (width 1) (layer B.Cu) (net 5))
 (segment (start 104.735 134.62) (end 104.735 131.62) (width 1) (layer B.Cu) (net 5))
 (segment (start 86.36 111.76) (end 86.36 110.49) (width 1) (layer B.Cu) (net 5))
 (segment (start 83.82 115.57) (end 83.82 114.3) (width 1) (layer B.Cu) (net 5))
 (segment (start 83.82 114.3) (end 86.36 111.76) (width 1) (layer B.Cu) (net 5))
 (segment (start 118.5 124.42) (end 121.5 124.42) (width 1) (layer B.Cu) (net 16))
 (segment (start 107.99 124.42) (end 118.5 124.42) (width 1) (layer B.Cu) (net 16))
 (segment (start 96.52 110.49) (end 96.52 113.03) (width 1) (layer B.Cu) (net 16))
 (segment (start 96.52 113.03) (end 107.95 124.46) (width 1) (layer B.Cu) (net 16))
 (segment (start 99.06 110.49) (end 99.06 111.49) (width 1) (layer B.Cu) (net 17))
 (segment (start 99.06 113.3475) (end 99.06 110.49) (width 1) (layer B.Cu) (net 17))
 (segment (start 121.5 119.42) (end 105.1325 119.42) (width 1) (layer B.Cu) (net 17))
 (segment (start 105.1325 119.42) (end 99.06 113.3475) (width 1) (layer B.Cu) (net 17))
 (segment (start 73.66 99.695) (end 73.66 102.87) (width 1) (layer B.Cu) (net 10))
 (segment (start 86.36 55.88) (end 82.55 59.69) (width 1) (layer B.Cu) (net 10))
 (segment (start 86.36 53.34) (end 86.36 55.88) (width 1) (layer B.Cu) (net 10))
 (segment (start 82.55 59.69) (end 82.55 74.295) (width 1) (layer B.Cu) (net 10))
 (segment (start 82.55 74.295) (end 76.2 80.645) (width 1) (layer B.Cu) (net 10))
 (segment (start 76.2 80.645) (end 76.2 97.155) (width 1) (layer B.Cu) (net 10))
 (segment (start 76.2 97.155) (end 73.66 99.695) (width 1) (layer B.Cu) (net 10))
 (segment (start 86.36 50.34) (end 86.36 53.34) (width 1) (layer B.Cu) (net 10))
 (segment (start 86.36 45.72) (end 86.36 50.34) (width 1) (layer B.Cu) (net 10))
 (segment (start 74.93 38.1) (end 78.74 38.1) (width 1) (layer B.Cu) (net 10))
 (segment (start 78.74 38.1) (end 86.36 45.72) (width 1) (layer B.Cu) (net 10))
 (segment (start 71.12 102.87) (end 71.12 103.87) (width 1) (layer B.Cu) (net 9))
 (segment (start 71.12 86.36) (end 70.12 86.36) (width 1) (layer B.Cu) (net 9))
 (segment (start 71.12 86.36) (end 71.96293 86.36) (width 1) (layer B.Cu) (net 9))
 (segment (start 71.12 98.7425) (end 71.12 102.87) (width 1) (layer B.Cu) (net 9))
 (segment (start 74.295 95.5675) (end 71.12 98.7425) (width 1) (layer B.Cu) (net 9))
 (segment (start 71.12 86.36) (end 74.295 89.535) (width 1) (layer B.Cu) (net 9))
 (segment (start 74.295 89.535) (end 74.295 95.5675) (width 1) (layer B.Cu) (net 9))
 (segment (start 88.9 56.34) (end 88.9 53.34) (width 1) (layer B.Cu) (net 9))
 (segment (start 85.09 60.15) (end 88.9 56.34) (width 1) (layer B.Cu) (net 9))
 (segment (start 85.09 75.565) (end 85.09 60.15) (width 1) (layer B.Cu) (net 9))
 (segment (start 81.28 86.36) (end 81.28 79.375) (width 1) (layer B.Cu) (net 9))
 (segment (start 81.28 79.375) (end 85.09 75.565) (width 1) (layer B.Cu) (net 9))
 (segment (start 88.9 50.34) (end 88.9 53.34) (width 1) (layer B.Cu) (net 9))
 (segment (start 88.9 45.085) (end 88.9 50.34) (width 1) (layer B.Cu) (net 9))
 (segment (start 74.93 35.56) (end 79.375 35.56) (width 1) (layer B.Cu) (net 9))
 (segment (start 79.375 35.56) (end 88.9 45.085) (width 1) (layer B.Cu) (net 9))
 (segment (start 98.425 53.34) (end 93.98 53.34) (width 1) (layer B.Cu) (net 18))
 (segment (start 93.94 61.42) (end 93.94 58.42) (width 1) (layer B.Cu) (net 18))
 (segment (start 93.94 62.19) (end 93.94 61.42) (width 1) (layer B.Cu) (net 18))
 (segment (start 92.075 64.135) (end 93.98 62.23) (width 1) (layer B.Cu) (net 18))
 (segment (start 93.98 62.23) (end 93.94 62.19) (width 1) (layer B.Cu) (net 18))
 (segment (start 93.94 53.38) (end 93.98 53.34) (width 1) (layer B.Cu) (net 18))
 (segment (start 93.94 58.42) (end 93.94 53.38) (width 1) (layer B.Cu) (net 18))
 (segment (start 63.5 41.656) (end 63.545167 41.701167) (width 1) (layer B.Cu) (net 8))
 (segment (start 56.515 111.76) (end 56.515 42.545) (width 1) (layer B.Cu) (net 8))
 (segment (start 58.42 113.665) (end 56.515 111.76) (width 1) (layer B.Cu) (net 8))
 (segment (start 78.105 113.665) (end 58.42 113.665) (width 1) (layer B.Cu) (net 8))
 (segment (start 78.74 110.49) (end 78.74 113.03) (width 1) (layer B.Cu) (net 8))
 (segment (start 78.74 113.03) (end 78.105 113.665) (width 1) (layer B.Cu) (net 8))
 (segment (start 107.95 110.49) (end 104.14 110.49) (width 1) (layer B.Cu) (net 7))
 (segment (start 111.125 107.315) (end 107.95 110.49) (width 1) (layer B.Cu) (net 7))
 (segment (start 111.125 47.895) (end 111.125 107.315) (width 1) (layer B.Cu) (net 7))
 (segment (start 117.11 41.91) (end 111.125 47.895) (width 1) (layer B.Cu) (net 7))
 (segment (start 118.11 41.91) (end 117.11 41.91) (width 1) (layer B.Cu) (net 7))
 (segment (start 110.76 139.7) (end 106.22 144.24) (width 1.27) (layer B.Cu) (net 3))
 (segment (start 111.76 139.7) (end 110.76 139.7) (width 1.27) (layer B.Cu) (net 3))
 (segment (start 116.38 139.7) (end 121.5 134.58) (width 1.27) (layer B.Cu) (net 3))
 (segment (start 111.76 139.7) (end 116.38 139.7) (width 1.27) (layer B.Cu) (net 3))
 (segment (start 102.87 144.24) (end 106.22 144.24) (width 1.27) (layer B.Cu) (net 3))
 (segment (start 102.87 141.645) (end 100.925 139.7) (width 1) (layer B.Cu) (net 3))
 (segment (start 102.87 144.945) (end 102.87 141.645) (width 1) (layer B.Cu) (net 3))
 (segment (start 102.87 166.945) (end 102.87 169.945) (width 1) (layer B.Cu) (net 6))
 (segment (start 102.87 156.21) (end 102.87 166.945) (width 1) (layer B.Cu) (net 6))
 (segment (start 121.5 149.74) (end 109.34 149.74) (width 1) (layer B.Cu) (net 6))
 (segment (start 109.34 149.74) (end 102.87 156.21) (width 1) (layer B.Cu) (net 6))
 (segment (start 106.8 129.42) (end 106.68 129.54) (width 1) (layer B.Cu) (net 15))
 (segment (start 121.5 129.42) (end 106.8 129.42) (width 1) (layer B.Cu) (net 15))
 (segment (start 121.5 144.74) (end 121.5 139.74) (width 1.27) (layer B.Cu) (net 19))
 (segment (start 116.245 114.26) (end 121.5 114.26) (width 1) (layer B.Cu) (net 12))
 (segment (start 114.3 112.315) (end 116.245 114.26) (width 1) (layer B.Cu) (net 12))
 (segment (start 114.3 97.79) (end 114.3 112.315) (width 1) (layer B.Cu) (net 12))
 (segment (start 89.535 93.345) (end 90.17 92.71) (width 1) (layer B.Cu) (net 11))
 (segment (start 81.28 93.345) (end 89.535 93.345) (width 1) (layer B.Cu) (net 11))
 (segment (start 66.04 100.33) (end 66.04 98.425) (width 1) (layer B.Cu) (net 2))
 (segment (start 66.04 98.425) (end 71.12 93.345) (width 1) (layer B.Cu) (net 2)))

